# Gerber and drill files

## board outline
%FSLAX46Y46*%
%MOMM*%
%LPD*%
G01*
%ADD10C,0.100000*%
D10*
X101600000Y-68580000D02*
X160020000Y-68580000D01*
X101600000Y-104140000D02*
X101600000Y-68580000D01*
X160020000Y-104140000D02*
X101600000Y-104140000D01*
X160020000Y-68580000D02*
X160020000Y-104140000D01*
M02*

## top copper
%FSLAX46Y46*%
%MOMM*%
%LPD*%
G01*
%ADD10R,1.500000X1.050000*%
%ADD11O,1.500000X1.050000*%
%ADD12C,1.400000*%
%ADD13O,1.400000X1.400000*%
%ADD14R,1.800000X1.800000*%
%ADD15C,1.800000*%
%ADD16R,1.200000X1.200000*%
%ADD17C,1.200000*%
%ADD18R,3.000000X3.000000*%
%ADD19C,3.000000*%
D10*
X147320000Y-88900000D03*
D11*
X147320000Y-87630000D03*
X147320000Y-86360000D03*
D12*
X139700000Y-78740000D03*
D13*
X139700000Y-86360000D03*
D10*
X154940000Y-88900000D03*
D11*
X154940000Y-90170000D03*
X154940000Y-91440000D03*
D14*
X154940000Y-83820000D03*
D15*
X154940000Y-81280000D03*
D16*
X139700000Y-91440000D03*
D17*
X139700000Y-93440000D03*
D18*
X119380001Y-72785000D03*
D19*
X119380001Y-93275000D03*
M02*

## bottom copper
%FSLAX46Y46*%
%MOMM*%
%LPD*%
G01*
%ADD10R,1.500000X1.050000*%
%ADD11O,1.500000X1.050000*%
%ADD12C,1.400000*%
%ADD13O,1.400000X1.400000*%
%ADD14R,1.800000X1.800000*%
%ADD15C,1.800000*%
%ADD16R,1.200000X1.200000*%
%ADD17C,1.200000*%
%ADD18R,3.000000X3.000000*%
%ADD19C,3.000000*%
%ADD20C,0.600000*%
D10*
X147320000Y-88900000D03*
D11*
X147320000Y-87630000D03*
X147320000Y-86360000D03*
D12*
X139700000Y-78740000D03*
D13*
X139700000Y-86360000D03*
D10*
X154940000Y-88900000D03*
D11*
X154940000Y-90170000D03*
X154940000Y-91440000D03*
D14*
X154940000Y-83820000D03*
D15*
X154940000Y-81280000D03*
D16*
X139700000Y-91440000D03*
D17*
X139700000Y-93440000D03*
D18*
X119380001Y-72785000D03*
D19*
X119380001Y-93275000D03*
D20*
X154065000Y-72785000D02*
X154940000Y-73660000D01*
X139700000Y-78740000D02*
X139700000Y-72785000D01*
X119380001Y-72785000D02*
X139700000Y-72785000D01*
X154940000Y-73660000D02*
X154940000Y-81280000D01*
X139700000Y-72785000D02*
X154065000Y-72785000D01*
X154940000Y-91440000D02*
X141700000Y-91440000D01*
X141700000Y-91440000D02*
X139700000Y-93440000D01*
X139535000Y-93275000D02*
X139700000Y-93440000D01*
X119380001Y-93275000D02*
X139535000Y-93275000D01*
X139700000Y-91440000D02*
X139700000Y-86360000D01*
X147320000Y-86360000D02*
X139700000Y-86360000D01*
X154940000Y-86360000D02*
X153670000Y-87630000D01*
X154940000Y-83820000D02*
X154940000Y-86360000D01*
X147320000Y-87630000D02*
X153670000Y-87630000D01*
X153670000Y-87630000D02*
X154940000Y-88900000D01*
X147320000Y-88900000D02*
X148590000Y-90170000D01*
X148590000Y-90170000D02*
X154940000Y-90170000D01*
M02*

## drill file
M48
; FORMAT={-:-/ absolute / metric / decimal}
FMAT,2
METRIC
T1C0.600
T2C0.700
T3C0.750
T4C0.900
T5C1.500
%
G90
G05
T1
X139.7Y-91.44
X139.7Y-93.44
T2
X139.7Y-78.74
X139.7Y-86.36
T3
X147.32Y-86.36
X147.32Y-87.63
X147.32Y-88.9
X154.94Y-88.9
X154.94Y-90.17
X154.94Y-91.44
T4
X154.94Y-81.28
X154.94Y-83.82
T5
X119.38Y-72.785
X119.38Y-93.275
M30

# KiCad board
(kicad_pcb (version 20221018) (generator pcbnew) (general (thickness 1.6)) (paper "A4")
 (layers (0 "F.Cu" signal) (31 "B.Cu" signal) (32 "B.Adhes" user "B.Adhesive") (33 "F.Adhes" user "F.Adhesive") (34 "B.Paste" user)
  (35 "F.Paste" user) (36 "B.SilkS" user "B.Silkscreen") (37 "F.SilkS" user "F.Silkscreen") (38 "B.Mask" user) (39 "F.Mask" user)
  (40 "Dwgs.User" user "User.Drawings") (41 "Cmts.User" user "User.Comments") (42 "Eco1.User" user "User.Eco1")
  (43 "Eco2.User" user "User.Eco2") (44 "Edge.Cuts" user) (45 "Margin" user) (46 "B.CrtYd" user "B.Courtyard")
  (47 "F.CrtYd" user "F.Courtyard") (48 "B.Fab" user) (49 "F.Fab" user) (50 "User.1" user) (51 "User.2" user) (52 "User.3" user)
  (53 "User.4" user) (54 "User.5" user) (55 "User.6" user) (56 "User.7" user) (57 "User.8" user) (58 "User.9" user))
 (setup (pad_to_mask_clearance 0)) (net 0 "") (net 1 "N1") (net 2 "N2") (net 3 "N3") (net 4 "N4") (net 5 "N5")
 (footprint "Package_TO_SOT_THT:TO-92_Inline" (layer "F.Cu") (at 147.32 88.9 90)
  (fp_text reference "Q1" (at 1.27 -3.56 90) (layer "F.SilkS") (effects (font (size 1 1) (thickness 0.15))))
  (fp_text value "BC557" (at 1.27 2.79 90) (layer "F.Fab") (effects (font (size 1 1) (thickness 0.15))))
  (pad "1" thru_hole rect (at 0 0 90) (size 1.05 1.5) (drill 0.75) (layers "*.Cu" "*.Mask") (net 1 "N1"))
  (pad "2" thru_hole oval (at 1.27 0 90) (size 1.05 1.5) (drill 0.75) (layers "*.Cu" "*.Mask") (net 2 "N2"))
  (pad "3" thru_hole oval (at 2.54 0 90) (size 1.05 1.5) (drill 0.75) (layers "*.Cu" "*.Mask") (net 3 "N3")))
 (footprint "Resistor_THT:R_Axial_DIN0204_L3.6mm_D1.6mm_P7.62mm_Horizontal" (layer "F.Cu") (at 139.7 78.74 -90)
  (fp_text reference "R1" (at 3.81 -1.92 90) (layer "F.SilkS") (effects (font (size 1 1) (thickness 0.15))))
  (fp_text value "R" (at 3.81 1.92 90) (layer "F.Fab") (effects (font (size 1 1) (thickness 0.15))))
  (pad "1" thru_hole circle (at 0 0 270) (size 1.4 1.4) (drill 0.7) (layers "*.Cu" "*.Mask") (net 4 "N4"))
  (pad "2" thru_hole oval (at 7.62 0 270) (size 1.4 1.4) (drill 0.7) (layers "*.Cu" "*.Mask") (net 3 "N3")))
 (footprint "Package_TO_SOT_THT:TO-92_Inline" (layer "F.Cu") (at 154.94 88.9 -90)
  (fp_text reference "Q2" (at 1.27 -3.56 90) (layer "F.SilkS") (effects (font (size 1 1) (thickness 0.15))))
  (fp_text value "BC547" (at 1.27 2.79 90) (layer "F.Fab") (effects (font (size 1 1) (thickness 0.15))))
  (pad "1" thru_hole rect (at 0 0 270) (size 1.05 1.5) (drill 0.75) (layers "*.Cu" "*.Mask") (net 2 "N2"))
  (pad "2" thru_hole oval (at 1.27 0 270) (size 1.05 1.5) (drill 0.75) (layers "*.Cu" "*.Mask") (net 1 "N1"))
  (pad "3" thru_hole oval (at 2.54 0 270) (size 1.05 1.5) (drill 0.75) (layers "*.Cu" "*.Mask") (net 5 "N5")))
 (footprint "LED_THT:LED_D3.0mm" (layer "F.Cu") (at 154.94 83.82 90)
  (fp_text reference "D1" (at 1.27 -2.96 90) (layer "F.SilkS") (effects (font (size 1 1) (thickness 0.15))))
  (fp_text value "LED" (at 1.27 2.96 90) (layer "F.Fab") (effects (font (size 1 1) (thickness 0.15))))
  (pad "1" thru_hole rect (at 0 0 90) (size 1.8 1.8) (drill 0.9) (layers "*.Cu" "*.Mask") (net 2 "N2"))
  (pad "2" thru_hole circle (at 2.54 0 90) (size 1.8 1.8) (drill 0.9) (layers "*.Cu" "*.Mask") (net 4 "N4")))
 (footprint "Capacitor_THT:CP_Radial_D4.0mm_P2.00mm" (layer "F.Cu") (at 139.7 91.44 -90)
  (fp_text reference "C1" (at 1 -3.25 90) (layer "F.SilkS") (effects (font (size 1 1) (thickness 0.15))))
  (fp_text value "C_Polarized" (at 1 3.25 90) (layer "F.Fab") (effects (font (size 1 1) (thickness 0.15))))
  (pad "1" thru_hole rect (at 0 0 270) (size 1.2 1.2) (drill 0.6) (layers "*.Cu" "*.Mask") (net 3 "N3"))
  (pad "2" thru_hole circle (at 2 0 270) (size 1.2 1.2) (drill 0.6) (layers "*.Cu" "*.Mask") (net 5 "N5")))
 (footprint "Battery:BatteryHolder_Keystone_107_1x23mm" (layer "F.Cu") (at 119.380001 72.785 -90)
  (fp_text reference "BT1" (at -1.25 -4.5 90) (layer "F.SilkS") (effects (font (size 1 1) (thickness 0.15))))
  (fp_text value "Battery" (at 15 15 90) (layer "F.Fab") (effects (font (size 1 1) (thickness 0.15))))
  (pad "1" thru_hole rect (at 0 0 270) (size 3 3) (drill 1.5) (layers "*.Cu" "*.Mask") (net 4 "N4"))
  (pad "2" thru_hole circle (at 20.49 0 270) (size 3 3) (drill 1.5) (layers "*.Cu" "*.Mask") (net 5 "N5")))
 (gr_line (start 101.6 68.58) (end 160.02 68.58) (stroke (width 0.1) (type default)) (layer "Edge.Cuts"))
 (gr_line (start 101.6 104.14) (end 101.6 68.58) (stroke (width 0.1) (type default)) (layer "Edge.Cuts"))
 (gr_line (start 160.02 104.14) (end 101.6 104.14) (stroke (width 0.1) (type default)) (layer "Edge.Cuts"))
 (gr_line (start 160.02 68.58) (end 160.02 104.14) (stroke (width 0.1) (type default)) (layer "Edge.Cuts"))
 (segment (start 154.065 72.785) (end 154.94 73.66) (width 0.6) (layer "B.Cu") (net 4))
 (segment (start 139.7 78.74) (end 139.7 72.785) (width 0.6) (layer "B.Cu") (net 4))
 (segment (start 119.380001 72.785) (end 139.7 72.785) (width 0.6) (layer "B.Cu") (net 4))
 (segment (start 154.94 73.66) (end 154.94 81.28) (width 0.6) (layer "B.Cu") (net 4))
 (segment (start 139.7 72.785) (end 154.065 72.785) (width 0.6) (layer "B.Cu") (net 4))
 (segment (start 154.94 91.44) (end 141.7 91.44) (width 0.6) (layer "B.Cu") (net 5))
 (segment (start 141.7 91.44) (end 139.7 93.44) (width 0.6) (layer "B.Cu") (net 5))
 (segment (start 139.535 93.275) (end 139.7 93.44) (width 0.6) (layer "B.Cu") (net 5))
 (segment (start 119.380001 93.275) (end 139.535 93.275) (width 0.6) (layer "B.Cu") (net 5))
 (segment (start 139.7 91.44) (end 139.7 86.36) (width 0.6) (layer "B.Cu") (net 3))
 (segment (start 147.32 86.36) (end 139.7 86.36) (width 0.6) (layer "B.Cu") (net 3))
 (segment (start 154.94 86.36) (end 153.67 87.63) (width 0.6) (layer "B.Cu") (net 2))
 (segment (start 154.94 83.82) (end 154.94 86.36) (width 0.6) (layer "B.Cu") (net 2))
 (segment (start 147.32 87.63) (end 153.67 87.63) (width 0.6) (layer "B.Cu") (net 2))
 (segment (start 153.67 87.63) (end 154.94 88.9) (width 0.6) (layer "B.Cu") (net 2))
 (segment (start 147.32 88.9) (end 148.59 90.17) (width 0.6) (layer "B.Cu") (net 1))
 (segment (start 148.59 90.17) (end 154.94 90.17) (width 0.6) (layer "B.Cu") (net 1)))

